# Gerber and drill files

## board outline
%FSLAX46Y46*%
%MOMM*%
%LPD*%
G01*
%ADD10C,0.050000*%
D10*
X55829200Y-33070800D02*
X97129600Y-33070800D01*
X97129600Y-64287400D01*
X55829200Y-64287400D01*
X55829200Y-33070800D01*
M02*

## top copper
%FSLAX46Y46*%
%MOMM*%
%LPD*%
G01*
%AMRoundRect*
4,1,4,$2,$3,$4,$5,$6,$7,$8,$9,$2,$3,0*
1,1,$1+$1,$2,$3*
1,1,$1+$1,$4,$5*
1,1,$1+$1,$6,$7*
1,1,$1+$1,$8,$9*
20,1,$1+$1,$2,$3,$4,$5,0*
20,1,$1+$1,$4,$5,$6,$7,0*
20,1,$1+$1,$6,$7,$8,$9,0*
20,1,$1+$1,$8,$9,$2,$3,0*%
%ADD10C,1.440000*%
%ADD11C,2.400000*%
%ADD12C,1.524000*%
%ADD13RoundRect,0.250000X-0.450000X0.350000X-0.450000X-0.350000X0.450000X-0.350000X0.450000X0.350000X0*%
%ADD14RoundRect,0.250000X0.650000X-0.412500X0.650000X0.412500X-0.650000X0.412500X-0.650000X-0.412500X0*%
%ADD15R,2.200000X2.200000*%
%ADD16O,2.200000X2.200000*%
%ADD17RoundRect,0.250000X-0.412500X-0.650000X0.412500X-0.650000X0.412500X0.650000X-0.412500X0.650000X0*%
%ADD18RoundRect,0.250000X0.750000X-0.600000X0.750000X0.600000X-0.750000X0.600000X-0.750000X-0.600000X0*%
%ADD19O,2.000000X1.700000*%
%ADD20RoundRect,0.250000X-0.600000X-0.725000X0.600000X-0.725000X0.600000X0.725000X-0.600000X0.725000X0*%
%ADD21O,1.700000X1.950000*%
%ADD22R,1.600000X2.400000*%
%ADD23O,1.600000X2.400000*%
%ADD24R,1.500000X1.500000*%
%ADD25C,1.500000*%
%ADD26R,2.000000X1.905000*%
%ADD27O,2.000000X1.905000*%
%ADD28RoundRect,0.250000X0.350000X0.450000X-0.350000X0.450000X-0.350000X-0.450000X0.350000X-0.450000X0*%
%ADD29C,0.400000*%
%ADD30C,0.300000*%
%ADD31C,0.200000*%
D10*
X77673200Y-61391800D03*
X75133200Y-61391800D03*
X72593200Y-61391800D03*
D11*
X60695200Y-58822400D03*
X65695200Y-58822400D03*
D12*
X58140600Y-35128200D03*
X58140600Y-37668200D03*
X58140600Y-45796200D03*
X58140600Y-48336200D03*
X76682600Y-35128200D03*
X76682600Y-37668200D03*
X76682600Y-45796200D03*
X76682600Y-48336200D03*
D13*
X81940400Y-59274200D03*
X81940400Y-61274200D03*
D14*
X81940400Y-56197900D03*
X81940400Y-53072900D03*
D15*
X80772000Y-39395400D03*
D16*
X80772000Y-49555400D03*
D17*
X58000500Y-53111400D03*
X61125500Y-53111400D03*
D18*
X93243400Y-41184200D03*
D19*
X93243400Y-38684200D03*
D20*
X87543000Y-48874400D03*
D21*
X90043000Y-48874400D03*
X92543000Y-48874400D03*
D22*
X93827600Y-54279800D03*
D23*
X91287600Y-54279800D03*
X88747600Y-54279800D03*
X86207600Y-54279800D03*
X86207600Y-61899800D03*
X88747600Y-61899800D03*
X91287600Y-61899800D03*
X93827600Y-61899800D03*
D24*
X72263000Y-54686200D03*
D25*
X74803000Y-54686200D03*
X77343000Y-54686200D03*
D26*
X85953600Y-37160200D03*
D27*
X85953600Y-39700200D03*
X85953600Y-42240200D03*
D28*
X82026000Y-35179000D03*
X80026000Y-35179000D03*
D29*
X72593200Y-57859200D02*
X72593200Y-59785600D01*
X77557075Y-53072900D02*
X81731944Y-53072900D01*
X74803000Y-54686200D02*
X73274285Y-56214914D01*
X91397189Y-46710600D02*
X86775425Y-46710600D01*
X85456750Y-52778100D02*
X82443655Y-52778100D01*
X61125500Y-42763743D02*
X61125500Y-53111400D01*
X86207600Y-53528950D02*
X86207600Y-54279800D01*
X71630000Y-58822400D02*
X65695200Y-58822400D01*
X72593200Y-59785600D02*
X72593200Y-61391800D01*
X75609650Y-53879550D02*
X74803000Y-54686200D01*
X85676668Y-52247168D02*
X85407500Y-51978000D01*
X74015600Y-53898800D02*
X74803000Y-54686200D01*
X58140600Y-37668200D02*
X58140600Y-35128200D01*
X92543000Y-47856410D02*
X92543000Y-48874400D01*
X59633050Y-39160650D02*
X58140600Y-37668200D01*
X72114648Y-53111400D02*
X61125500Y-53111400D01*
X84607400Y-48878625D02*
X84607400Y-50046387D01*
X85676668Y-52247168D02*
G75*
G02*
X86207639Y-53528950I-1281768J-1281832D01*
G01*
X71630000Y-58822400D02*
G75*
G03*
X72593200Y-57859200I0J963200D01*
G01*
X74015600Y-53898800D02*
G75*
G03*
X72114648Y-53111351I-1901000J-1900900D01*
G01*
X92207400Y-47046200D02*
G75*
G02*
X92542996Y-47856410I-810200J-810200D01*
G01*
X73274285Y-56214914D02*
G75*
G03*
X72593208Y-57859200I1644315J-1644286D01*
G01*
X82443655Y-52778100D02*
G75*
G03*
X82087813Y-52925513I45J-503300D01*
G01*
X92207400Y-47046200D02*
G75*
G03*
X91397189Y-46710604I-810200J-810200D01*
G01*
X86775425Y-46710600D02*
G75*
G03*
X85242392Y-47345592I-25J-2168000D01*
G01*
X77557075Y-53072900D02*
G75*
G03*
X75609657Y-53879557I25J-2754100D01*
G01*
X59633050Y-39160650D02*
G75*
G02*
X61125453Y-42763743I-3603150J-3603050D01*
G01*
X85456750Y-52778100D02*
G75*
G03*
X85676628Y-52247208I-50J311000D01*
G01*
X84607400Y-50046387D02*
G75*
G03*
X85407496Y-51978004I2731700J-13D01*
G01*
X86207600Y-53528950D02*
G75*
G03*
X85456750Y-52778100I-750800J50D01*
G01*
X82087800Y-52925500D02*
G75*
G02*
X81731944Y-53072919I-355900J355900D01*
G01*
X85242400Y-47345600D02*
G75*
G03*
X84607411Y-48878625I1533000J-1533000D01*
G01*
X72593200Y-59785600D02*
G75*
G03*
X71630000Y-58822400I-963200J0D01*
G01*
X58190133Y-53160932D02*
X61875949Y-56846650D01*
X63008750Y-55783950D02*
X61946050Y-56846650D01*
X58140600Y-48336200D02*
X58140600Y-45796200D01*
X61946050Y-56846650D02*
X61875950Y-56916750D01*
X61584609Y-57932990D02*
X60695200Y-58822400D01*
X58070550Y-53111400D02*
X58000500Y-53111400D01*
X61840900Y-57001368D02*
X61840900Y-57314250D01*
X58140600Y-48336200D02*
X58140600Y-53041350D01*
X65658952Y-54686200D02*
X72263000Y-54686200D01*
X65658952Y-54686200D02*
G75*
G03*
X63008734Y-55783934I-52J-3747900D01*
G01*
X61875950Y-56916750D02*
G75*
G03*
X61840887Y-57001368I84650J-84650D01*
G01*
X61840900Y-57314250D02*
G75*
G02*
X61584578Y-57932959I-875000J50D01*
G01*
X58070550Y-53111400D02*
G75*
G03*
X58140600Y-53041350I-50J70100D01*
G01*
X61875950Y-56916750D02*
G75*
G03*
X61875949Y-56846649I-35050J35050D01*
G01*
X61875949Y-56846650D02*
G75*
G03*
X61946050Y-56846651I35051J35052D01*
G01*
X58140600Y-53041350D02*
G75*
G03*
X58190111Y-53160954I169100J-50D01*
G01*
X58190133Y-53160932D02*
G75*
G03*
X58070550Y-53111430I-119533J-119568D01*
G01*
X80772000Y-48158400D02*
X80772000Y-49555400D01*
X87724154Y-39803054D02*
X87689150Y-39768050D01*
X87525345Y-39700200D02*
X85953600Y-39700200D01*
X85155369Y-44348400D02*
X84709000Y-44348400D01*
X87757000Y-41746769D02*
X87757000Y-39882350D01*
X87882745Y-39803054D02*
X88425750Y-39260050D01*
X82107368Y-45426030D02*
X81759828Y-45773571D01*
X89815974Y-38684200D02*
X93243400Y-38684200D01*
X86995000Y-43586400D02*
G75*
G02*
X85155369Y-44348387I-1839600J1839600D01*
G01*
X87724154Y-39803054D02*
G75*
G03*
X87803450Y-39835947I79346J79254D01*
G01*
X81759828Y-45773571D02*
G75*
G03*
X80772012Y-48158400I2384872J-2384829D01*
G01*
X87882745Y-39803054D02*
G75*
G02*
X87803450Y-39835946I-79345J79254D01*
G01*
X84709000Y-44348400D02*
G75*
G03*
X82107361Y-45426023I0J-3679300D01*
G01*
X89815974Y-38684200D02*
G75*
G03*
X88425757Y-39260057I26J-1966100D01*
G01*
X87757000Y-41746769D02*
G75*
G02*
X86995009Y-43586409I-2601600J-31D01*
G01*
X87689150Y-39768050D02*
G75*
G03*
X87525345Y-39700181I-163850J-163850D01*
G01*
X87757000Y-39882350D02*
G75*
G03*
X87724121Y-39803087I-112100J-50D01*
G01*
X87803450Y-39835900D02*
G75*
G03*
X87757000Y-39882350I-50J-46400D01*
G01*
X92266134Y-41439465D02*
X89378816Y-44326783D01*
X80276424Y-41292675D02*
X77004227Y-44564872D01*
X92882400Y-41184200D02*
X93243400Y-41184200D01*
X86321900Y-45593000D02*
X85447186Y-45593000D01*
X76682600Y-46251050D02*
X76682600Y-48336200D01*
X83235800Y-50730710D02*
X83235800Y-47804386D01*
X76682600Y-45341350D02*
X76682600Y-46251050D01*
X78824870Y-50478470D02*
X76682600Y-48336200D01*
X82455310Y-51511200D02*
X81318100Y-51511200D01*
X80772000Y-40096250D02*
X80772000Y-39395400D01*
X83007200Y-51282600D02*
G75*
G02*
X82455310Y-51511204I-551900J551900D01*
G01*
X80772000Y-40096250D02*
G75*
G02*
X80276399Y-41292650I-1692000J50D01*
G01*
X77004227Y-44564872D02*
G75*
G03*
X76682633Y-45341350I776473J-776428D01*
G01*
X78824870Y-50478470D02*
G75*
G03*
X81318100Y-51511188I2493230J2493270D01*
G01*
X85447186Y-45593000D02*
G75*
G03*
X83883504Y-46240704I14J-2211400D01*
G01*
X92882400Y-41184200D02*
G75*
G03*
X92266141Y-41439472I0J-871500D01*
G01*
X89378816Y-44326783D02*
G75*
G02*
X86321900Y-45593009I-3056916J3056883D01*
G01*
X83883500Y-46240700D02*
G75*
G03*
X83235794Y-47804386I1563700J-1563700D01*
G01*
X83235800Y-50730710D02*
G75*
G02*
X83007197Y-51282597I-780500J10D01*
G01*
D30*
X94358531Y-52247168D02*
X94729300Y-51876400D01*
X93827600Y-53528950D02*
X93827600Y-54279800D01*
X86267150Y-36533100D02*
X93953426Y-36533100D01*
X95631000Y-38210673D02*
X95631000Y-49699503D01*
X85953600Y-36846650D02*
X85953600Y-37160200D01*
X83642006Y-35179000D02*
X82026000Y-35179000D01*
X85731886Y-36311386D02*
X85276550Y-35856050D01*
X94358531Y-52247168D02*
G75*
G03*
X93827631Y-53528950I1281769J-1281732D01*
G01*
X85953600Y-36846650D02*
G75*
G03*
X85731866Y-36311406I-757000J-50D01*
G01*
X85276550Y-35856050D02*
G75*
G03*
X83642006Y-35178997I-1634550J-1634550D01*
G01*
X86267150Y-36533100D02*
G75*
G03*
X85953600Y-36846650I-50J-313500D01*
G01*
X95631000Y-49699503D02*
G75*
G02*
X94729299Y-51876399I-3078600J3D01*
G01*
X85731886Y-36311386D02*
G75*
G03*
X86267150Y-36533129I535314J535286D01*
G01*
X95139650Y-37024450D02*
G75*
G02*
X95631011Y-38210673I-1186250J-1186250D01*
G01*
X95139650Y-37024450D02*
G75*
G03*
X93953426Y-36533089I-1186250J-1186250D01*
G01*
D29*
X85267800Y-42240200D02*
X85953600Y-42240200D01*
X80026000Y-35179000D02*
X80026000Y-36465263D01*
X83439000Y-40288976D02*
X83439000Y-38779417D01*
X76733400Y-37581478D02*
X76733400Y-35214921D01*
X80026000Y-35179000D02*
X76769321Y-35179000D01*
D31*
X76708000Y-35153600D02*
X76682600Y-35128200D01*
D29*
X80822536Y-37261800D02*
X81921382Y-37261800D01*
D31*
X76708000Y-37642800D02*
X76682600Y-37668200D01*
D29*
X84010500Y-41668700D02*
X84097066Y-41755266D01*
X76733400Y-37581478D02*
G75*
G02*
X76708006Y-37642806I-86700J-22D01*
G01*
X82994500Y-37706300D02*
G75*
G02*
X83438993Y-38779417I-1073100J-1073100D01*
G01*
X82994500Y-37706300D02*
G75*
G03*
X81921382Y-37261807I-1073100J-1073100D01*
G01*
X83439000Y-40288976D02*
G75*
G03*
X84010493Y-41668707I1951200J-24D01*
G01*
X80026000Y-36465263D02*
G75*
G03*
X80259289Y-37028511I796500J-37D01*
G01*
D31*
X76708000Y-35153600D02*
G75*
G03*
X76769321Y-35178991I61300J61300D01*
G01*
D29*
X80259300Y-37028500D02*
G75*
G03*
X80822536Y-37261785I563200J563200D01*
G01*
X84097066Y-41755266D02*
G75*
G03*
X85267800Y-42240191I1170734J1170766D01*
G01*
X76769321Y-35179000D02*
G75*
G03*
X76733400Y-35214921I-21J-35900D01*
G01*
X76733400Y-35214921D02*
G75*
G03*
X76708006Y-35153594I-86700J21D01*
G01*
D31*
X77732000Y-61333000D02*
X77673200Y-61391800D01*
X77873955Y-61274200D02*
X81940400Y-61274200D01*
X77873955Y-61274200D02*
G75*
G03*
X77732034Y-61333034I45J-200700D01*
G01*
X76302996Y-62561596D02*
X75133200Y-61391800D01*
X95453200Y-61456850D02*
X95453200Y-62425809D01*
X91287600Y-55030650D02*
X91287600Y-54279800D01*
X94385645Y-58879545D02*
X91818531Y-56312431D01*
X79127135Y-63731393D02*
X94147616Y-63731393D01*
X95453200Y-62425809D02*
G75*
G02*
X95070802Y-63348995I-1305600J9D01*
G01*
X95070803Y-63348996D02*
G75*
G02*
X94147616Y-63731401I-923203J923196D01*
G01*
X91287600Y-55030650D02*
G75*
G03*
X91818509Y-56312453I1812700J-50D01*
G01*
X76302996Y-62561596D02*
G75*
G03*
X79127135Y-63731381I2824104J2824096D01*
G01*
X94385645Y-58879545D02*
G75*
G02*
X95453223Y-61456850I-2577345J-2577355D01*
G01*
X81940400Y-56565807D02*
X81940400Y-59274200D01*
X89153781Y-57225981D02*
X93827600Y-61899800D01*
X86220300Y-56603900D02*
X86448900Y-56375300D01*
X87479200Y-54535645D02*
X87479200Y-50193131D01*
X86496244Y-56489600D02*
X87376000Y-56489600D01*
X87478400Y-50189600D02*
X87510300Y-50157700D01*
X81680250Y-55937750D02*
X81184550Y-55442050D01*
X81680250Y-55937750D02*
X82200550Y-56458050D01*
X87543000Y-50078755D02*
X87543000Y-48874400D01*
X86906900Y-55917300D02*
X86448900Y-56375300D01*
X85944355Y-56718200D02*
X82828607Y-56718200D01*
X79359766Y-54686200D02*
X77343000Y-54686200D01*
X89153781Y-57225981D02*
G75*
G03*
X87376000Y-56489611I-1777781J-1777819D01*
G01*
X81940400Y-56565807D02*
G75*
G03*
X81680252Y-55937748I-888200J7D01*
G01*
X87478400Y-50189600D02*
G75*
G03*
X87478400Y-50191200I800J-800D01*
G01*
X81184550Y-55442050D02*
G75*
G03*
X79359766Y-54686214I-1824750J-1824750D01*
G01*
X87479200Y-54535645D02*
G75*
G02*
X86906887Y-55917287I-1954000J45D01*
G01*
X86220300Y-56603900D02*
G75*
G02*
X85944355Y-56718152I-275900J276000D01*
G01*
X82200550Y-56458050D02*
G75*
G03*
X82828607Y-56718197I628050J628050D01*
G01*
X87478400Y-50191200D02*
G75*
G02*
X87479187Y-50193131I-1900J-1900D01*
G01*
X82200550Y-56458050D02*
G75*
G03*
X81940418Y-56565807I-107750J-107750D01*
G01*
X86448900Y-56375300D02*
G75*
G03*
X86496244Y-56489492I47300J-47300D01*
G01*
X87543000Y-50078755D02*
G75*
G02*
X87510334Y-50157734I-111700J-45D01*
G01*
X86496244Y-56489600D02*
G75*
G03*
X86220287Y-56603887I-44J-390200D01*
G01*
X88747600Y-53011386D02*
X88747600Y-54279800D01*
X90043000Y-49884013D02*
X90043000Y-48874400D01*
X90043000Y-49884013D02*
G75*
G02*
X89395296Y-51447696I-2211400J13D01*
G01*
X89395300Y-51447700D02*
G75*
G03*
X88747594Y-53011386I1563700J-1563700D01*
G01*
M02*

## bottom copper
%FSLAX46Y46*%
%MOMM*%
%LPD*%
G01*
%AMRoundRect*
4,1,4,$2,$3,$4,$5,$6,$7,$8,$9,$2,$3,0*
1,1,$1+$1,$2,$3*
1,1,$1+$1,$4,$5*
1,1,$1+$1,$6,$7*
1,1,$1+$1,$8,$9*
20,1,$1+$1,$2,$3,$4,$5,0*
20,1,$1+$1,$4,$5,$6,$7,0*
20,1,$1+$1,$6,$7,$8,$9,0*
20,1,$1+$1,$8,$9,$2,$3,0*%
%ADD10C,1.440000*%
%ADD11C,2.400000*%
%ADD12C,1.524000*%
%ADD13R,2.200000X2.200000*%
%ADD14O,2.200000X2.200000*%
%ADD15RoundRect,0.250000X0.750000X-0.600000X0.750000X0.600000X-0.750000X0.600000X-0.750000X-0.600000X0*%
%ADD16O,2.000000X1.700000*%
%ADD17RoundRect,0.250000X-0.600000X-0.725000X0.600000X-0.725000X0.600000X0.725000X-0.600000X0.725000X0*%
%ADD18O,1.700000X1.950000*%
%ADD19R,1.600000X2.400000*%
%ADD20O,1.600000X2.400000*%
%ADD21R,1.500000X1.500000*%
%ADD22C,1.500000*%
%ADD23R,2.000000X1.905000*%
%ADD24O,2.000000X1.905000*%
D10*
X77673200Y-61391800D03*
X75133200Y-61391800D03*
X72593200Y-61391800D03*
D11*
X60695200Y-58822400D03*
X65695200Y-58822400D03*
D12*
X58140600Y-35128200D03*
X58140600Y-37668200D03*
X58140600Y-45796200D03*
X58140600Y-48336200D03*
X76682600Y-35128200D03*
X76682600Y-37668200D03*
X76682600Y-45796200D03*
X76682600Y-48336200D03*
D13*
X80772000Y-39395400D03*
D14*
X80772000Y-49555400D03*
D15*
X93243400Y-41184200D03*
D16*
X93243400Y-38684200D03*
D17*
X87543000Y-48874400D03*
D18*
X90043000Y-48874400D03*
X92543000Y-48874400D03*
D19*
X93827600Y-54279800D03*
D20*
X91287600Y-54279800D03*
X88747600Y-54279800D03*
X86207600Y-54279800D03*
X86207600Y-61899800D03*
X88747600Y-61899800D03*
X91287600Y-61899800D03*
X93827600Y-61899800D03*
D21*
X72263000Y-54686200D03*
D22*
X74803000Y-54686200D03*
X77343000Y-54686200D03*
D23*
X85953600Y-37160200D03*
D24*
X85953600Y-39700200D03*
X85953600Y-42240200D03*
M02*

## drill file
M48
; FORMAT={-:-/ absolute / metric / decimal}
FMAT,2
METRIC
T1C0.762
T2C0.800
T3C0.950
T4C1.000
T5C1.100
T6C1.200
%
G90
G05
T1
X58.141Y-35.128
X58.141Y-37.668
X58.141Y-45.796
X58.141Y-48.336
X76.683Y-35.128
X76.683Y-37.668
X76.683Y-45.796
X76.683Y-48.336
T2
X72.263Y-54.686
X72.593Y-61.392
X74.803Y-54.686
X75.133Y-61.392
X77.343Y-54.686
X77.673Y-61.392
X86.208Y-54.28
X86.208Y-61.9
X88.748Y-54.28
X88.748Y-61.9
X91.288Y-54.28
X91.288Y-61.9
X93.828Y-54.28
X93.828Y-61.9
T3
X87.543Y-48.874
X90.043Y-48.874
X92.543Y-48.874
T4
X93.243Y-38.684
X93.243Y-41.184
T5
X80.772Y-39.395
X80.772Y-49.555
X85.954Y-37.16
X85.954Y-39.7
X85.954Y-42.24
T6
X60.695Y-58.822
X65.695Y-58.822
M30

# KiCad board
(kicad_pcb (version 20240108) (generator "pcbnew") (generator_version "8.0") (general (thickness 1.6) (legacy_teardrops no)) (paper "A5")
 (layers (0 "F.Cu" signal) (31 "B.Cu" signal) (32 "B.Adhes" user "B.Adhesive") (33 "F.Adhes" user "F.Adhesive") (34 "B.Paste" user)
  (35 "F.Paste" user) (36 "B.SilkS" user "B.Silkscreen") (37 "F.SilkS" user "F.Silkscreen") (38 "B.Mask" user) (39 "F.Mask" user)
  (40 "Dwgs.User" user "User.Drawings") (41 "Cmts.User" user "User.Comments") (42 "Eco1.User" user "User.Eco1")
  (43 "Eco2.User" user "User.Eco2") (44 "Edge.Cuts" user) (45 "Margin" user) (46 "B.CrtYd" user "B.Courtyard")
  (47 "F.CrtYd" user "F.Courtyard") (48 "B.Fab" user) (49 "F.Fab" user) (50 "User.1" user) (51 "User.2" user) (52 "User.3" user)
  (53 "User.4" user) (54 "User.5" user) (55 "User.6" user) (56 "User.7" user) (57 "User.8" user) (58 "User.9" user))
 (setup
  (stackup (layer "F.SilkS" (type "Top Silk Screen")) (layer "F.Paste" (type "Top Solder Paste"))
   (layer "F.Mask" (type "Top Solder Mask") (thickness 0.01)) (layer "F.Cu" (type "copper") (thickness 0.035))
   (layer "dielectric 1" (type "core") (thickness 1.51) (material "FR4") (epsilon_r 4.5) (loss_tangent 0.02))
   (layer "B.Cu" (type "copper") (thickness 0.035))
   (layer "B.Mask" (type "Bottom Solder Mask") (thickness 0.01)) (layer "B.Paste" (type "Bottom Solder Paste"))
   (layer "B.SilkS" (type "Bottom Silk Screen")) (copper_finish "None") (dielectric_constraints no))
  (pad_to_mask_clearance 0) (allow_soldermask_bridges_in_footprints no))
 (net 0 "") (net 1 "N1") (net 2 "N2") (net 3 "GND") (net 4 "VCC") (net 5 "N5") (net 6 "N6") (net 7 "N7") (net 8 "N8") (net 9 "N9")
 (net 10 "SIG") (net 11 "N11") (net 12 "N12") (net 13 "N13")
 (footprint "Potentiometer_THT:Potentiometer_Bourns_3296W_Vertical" (layer "F.Cu") (at 77.6732 61.3918)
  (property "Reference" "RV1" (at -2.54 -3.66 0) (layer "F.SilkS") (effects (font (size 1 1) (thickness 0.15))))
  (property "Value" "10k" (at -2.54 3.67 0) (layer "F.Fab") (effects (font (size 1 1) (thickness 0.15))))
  (pad "1" thru_hole circle (at 0 0) (size 1.44 1.44) (drill 0.8) (layers "*.Cu" "*.Mask") (remove_unused_layers no) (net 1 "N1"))
  (pad "2" thru_hole circle (at -2.54 0) (size 1.44 1.44) (drill 0.8) (layers "*.Cu" "*.Mask") (remove_unused_layers no) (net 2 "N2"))
  (pad "3" thru_hole circle (at -5.08 0) (size 1.44 1.44) (drill 0.8) (layers "*.Cu" "*.Mask") (remove_unused_layers no) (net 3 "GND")))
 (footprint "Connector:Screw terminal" (layer "F.Cu") (at 63.1952 58.9224)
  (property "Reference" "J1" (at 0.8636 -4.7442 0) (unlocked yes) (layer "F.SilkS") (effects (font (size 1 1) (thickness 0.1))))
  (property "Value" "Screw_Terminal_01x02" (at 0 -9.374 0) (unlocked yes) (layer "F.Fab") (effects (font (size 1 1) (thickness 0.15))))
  (pad "1" thru_hole circle (at -2.5 -0.1) (size 2.4 2.4) (drill 1.2) (layers "*.Cu" "*.Mask") (remove_unused_layers no) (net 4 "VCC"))
  (pad "2" thru_hole circle (at 2.5 -0.1) (size 2.4 2.4) (drill 1.2) (layers "*.Cu" "*.Mask") (remove_unused_layers no) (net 3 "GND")))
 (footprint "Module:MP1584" (layer "F.Cu") (at 69.0626 41.2242)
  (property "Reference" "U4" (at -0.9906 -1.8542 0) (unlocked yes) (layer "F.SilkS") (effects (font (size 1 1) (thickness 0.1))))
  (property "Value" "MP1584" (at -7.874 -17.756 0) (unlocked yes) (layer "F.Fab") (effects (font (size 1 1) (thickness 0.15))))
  (pad "1" thru_hole circle (at -10.922 -6.096) (size 1.524 1.524) (drill 0.762) (layers "*.Cu" "*.Mask") (remove_unused_layers no)
   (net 3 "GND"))
  (pad "1" thru_hole circle (at -10.922 -3.556) (size 1.524 1.524) (drill 0.762) (layers "*.Cu" "*.Mask") (remove_unused_layers no)
   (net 3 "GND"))
  (pad "2" thru_hole circle (at -10.922 4.572) (size 1.524 1.524) (drill 0.762) (layers "*.Cu" "*.Mask") (remove_unused_layers no)
   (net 4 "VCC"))
  (pad "2" thru_hole circle (at -10.922 7.112) (size 1.524 1.524) (drill 0.762) (layers "*.Cu" "*.Mask") (remove_unused_layers no)
   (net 4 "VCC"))
  (pad "3" thru_hole circle (at 7.62 -6.096) (size 1.524 1.524) (drill 0.762) (layers "*.Cu" "*.Mask") (remove_unused_layers no)
   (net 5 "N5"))
  (pad "3" thru_hole circle (at 7.62 -3.556) (size 1.524 1.524) (drill 0.762) (layers "*.Cu" "*.Mask") (remove_unused_layers no)
   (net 5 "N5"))
  (pad "4" thru_hole circle (at 7.62 4.572) (size 1.524 1.524) (drill 0.762) (layers "*.Cu" "*.Mask") (remove_unused_layers no) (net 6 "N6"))
  (pad "4" thru_hole circle (at 7.62 7.112) (size 1.524 1.524) (drill 0.762) (layers "*.Cu" "*.Mask") (remove_unused_layers no) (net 6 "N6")))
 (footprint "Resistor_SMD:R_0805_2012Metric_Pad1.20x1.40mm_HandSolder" (layer "F.Cu") (at 81.9404 60.2742 -90)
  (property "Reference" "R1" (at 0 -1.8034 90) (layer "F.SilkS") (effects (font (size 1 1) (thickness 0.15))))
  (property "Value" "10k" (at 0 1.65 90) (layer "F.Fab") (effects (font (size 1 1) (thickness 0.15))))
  (pad "1" smd roundrect (at -1 0 270) (size 1.2 1.4) (layers "F.Cu" "F.Paste" "F.Mask") (roundrect_rratio 0.208333) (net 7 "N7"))
  (pad "2" smd roundrect (at 1 0 270) (size 1.2 1.4) (layers "F.Cu" "F.Paste" "F.Mask") (roundrect_rratio 0.208333) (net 1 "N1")))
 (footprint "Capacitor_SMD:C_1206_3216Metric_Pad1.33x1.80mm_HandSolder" (layer "F.Cu") (at 81.9404 54.6354 90)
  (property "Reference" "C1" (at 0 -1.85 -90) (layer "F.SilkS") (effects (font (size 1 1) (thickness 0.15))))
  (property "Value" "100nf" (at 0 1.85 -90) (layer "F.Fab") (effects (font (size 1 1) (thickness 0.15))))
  (pad "1" smd roundrect (at -1.5625 0 90) (size 1.325 1.8) (layers "F.Cu" "F.Paste" "F.Mask") (roundrect_rratio 0.188679) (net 7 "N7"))
  (pad "2" smd roundrect (at 1.5625 0 90) (size 1.325 1.8) (layers "F.Cu" "F.Paste" "F.Mask") (roundrect_rratio 0.188679) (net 3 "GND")))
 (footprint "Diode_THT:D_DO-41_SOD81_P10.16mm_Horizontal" (layer "F.Cu") (at 80.772 39.3954 -90)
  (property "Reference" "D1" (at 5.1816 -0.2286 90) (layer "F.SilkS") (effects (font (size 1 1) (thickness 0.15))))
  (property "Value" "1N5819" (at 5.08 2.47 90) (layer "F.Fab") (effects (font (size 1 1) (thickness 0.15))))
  (pad "1" thru_hole rect (at 0 0 270) (size 2.2 2.2) (drill 1.1) (layers "*.Cu" "*.Mask") (remove_unused_layers no) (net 6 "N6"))
  (pad "2" thru_hole oval (at 10.16 0 270) (size 2.2 2.2) (drill 1.1) (layers "*.Cu" "*.Mask") (remove_unused_layers no) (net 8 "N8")))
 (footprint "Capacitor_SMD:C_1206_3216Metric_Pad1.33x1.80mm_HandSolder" (layer "F.Cu") (at 59.563 53.1114)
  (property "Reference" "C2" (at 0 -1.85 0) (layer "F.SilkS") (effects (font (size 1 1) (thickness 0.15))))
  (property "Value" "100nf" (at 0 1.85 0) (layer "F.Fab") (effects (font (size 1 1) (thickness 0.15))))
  (pad "1" smd roundrect (at -1.5625 0) (size 1.325 1.8) (layers "F.Cu" "F.Paste" "F.Mask") (roundrect_rratio 0.188679) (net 4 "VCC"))
  (pad "2" smd roundrect (at 1.5625 0) (size 1.325 1.8) (layers "F.Cu" "F.Paste" "F.Mask") (roundrect_rratio 0.188679) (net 3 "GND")))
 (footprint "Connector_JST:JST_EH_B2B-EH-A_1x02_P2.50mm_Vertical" (layer "F.Cu") (at 93.2434 41.1842 90)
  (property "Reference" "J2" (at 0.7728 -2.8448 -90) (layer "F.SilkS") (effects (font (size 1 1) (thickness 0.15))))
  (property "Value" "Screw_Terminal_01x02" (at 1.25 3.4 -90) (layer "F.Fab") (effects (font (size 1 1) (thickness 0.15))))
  (pad "1" thru_hole roundrect (at 0 0 90) (size 1.7 2) (drill 1) (layers "*.Cu" "*.Mask") (remove_unused_layers no)
   (roundrect_rratio 0.147059) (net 6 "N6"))
  (pad "2" thru_hole oval (at 2.5 0 90) (size 1.7 2) (drill 1) (layers "*.Cu" "*.Mask") (remove_unused_layers no) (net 8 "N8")))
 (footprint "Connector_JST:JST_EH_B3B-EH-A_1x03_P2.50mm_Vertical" (layer "F.Cu") (at 87.543 48.8744)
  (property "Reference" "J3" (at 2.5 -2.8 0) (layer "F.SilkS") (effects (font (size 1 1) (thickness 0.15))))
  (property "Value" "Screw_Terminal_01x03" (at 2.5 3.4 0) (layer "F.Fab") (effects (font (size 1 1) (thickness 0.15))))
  (pad "1" thru_hole roundrect (at 0 0) (size 1.7 1.95) (drill 0.95) (layers "*.Cu" "*.Mask") (remove_unused_layers no)
   (roundrect_rratio 0.147059) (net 7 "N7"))
  (pad "2" thru_hole oval (at 2.5 0) (size 1.7 1.95) (drill 0.95) (layers "*.Cu" "*.Mask") (remove_unused_layers no) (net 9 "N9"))
  (pad "3" thru_hole oval (at 5 0) (size 1.7 1.95) (drill 0.95) (layers "*.Cu" "*.Mask") (remove_unused_layers no) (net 3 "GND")))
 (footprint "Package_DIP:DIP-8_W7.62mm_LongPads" (layer "F.Cu") (at 93.8276 54.2798 -90)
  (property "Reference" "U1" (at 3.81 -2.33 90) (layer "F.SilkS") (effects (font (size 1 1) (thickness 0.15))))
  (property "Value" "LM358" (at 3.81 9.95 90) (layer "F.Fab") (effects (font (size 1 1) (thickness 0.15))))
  (pad "1" thru_hole rect (at 0 0 270) (size 2.4 1.6) (drill 0.8) (layers "*.Cu" "*.Mask") (remove_unused_layers no) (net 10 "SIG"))
  (pad "2" thru_hole oval (at 0 2.54 270) (size 2.4 1.6) (drill 0.8) (layers "*.Cu" "*.Mask") (remove_unused_layers no) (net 2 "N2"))
  (pad "3" thru_hole oval (at 0 5.08 270) (size 2.4 1.6) (drill 0.8) (layers "*.Cu" "*.Mask") (remove_unused_layers no) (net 9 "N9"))
  (pad "4" thru_hole oval (at 0 7.62 270) (size 2.4 1.6) (drill 0.8) (layers "*.Cu" "*.Mask") (remove_unused_layers no) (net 3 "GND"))
  (pad "5" thru_hole oval (at 7.62 7.62 270) (size 2.4 1.6) (drill 0.8) (layers "*.Cu" "*.Mask") (remove_unused_layers no) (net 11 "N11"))
  (pad "6" thru_hole oval (at 7.62 5.08 270) (size 2.4 1.6) (drill 0.8) (layers "*.Cu" "*.Mask") (remove_unused_layers no) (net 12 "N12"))
  (pad "7" thru_hole oval (at 7.62 2.54 270) (size 2.4 1.6) (drill 0.8) (layers "*.Cu" "*.Mask") (remove_unused_layers no) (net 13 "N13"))
  (pad "8" thru_hole oval (at 7.62 0 270) (size 2.4 1.6) (drill 0.8) (layers "*.Cu" "*.Mask") (remove_unused_layers no) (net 7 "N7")))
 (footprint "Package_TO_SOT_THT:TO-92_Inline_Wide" (layer "F.Cu") (at 72.263 54.6862)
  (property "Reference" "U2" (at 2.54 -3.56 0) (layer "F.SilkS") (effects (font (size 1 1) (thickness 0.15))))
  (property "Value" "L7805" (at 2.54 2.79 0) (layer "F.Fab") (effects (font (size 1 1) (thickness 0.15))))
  (pad "1" thru_hole rect (at 0 0) (size 1.5 1.5) (drill 0.8) (layers "*.Cu" "*.Mask") (remove_unused_layers no) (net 4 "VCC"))
  (pad "2" thru_hole circle (at 2.54 0) (size 1.5 1.5) (drill 0.8) (layers "*.Cu" "*.Mask") (remove_unused_layers no) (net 3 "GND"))
  (pad "3" thru_hole circle (at 5.08 0) (size 1.5 1.5) (drill 0.8) (layers "*.Cu" "*.Mask") (remove_unused_layers no) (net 7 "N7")))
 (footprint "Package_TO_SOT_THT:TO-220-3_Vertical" (layer "F.Cu") (at 85.9536 37.1602 -90)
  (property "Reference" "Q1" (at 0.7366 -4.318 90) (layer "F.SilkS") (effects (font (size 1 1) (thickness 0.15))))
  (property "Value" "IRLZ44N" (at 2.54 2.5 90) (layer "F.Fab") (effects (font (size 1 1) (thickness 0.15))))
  (pad "1" thru_hole rect (at 0 0 270) (size 1.905 2) (drill 1.1) (layers "*.Cu" "*.Mask") (remove_unused_layers no) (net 10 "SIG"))
  (pad "2" thru_hole oval (at 2.54 0 270) (size 1.905 2) (drill 1.1) (layers "*.Cu" "*.Mask") (remove_unused_layers no) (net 8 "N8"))
  (pad "3" thru_hole oval (at 5.08 0 270) (size 1.905 2) (drill 1.1) (layers "*.Cu" "*.Mask") (remove_unused_layers no) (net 5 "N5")))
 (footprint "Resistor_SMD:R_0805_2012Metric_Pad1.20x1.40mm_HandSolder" (layer "F.Cu") (at 81.026 35.179 180)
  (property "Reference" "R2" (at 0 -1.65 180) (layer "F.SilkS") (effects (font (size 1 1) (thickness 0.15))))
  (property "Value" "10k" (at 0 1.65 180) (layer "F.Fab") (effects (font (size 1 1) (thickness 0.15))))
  (pad "1" smd roundrect (at -1 0 180) (size 1.2 1.4) (layers "F.Cu" "F.Paste" "F.Mask") (roundrect_rratio 0.208333) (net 10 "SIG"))
  (pad "2" smd roundrect (at 1 0 180) (size 1.2 1.4) (layers "F.Cu" "F.Paste" "F.Mask") (roundrect_rratio 0.208333) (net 5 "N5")))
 (gr_rect (start 55.8292 33.0708) (end 97.1296 64.2874) (stroke (width 0.05) (type default)) (fill none) (layer "Edge.Cuts"))
 (segment (start 72.5932 57.8592) (end 72.5932 59.7856) (width 0.4) (layer "F.Cu") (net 3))
 (segment (start 77.557075 53.0729) (end 81.731944 53.0729) (width 0.4) (layer "F.Cu") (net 3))
 (segment (start 74.803 54.6862) (end 73.274285 56.214914) (width 0.4) (layer "F.Cu") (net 3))
 (segment (start 91.397189 46.7106) (end 86.775425 46.7106) (width 0.4) (layer "F.Cu") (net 3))
 (segment (start 85.45675 52.7781) (end 82.443655 52.7781) (width 0.4) (layer "F.Cu") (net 3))
 (segment (start 61.1255 42.763743) (end 61.1255 53.1114) (width 0.4) (layer "F.Cu") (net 3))
 (segment (start 86.2076 53.52895) (end 86.2076 54.2798) (width 0.4) (layer "F.Cu") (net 3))
 (segment (start 71.63 58.8224) (end 65.6952 58.8224) (width 0.4) (layer "F.Cu") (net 3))
 (segment (start 72.5932 59.7856) (end 72.5932 61.3918) (width 0.4) (layer "F.Cu") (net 3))
 (segment (start 75.60965 53.87955) (end 74.803 54.6862) (width 0.4) (layer "F.Cu") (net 3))
 (segment (start 85.676668 52.247168) (end 85.4075 51.978) (width 0.4) (layer "F.Cu") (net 3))
 (segment (start 74.0156 53.8988) (end 74.803 54.6862) (width 0.4) (layer "F.Cu") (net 3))
 (segment (start 58.1406 37.6682) (end 58.1406 35.1282) (width 0.4) (layer "F.Cu") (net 3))
 (segment (start 92.543 47.85641) (end 92.543 48.8744) (width 0.4) (layer "F.Cu") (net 3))
 (segment (start 59.63305 39.16065) (end 58.1406 37.6682) (width 0.4) (layer "F.Cu") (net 3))
 (segment (start 72.114648 53.1114) (end 61.1255 53.1114) (width 0.4) (layer "F.Cu") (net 3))
 (segment (start 84.6074 48.878625) (end 84.6074 50.046387) (width 0.4) (layer "F.Cu") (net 3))
 (arc (start 85.676668 52.247168) (mid 86.069615 52.835254) (end 86.2076 53.52895) (width 0.4) (layer "F.Cu") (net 3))
 (arc (start 71.63 58.8224) (mid 72.311085 58.540285) (end 72.5932 57.8592) (width 0.4) (layer "F.Cu") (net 3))
 (arc (start 74.0156 53.8988) (mid 73.143435 53.316038) (end 72.114648 53.1114) (width 0.4) (layer "F.Cu") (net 3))
 (arc (start 92.2074 47.0462) (mid 92.45578 47.417927) (end 92.543 47.85641) (width 0.4) (layer "F.Cu") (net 3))
 (arc (start 73.274285 56.214914) (mid 72.770208 56.969319) (end 72.5932 57.8592) (width 0.4) (layer "F.Cu") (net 3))
 (arc (start 82.443655 52.7781) (mid 82.251067 52.816408) (end 82.0878 52.9255) (width 0.4) (layer "F.Cu") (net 3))
 (arc (start 92.2074 47.0462) (mid 91.835672 46.797819) (end 91.397189 46.7106) (width 0.4) (layer "F.Cu") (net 3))
 (arc (start 86.775425 46.7106) (mid 85.945757 46.875631) (end 85.2424 47.3456) (width 0.4) (layer "F.Cu") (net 3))
 (arc (start 77.557075 53.0729) (mid 76.503136 53.282541) (end 75.60965 53.87955) (width 0.4) (layer "F.Cu") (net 3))
 (arc (start 59.63305 39.16065) (mid 60.737624 40.813763) (end 61.1255 42.763743) (width 0.4) (layer "F.Cu") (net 3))
 (arc (start 85.45675 52.7781) (mid 85.744087 52.586106) (end 85.676668 52.247168) (width 0.4) (layer "F.Cu") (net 3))
 (arc (start 84.6074 50.046387) (mid 84.815339 51.091768) (end 85.4075 51.978) (width 0.4) (layer "F.Cu") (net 3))
 (arc (start 86.2076 53.52895) (mid 85.987681 52.998018) (end 85.45675 52.7781) (width 0.4) (layer "F.Cu") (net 3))
 (arc (start 82.0878 52.9255) (mid 81.924532 53.034591) (end 81.731944 53.0729) (width 0.4) (layer "F.Cu") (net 3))
 (arc (start 85.2424 47.3456) (mid 84.772431 48.048957) (end 84.6074 48.878625) (width 0.4) (layer "F.Cu") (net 3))
 (arc (start 72.5932 59.7856) (mid 72.311085 59.104514) (end 71.63 58.8224) (width 0.4) (layer "F.Cu") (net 3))
 (segment (start 58.190133 53.160932) (end 61.875949 56.84665) (width 0.4) (layer "F.Cu") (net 4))
 (segment (start 63.00875 55.78395) (end 61.94605 56.84665) (width 0.4) (layer "F.Cu") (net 4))
 (segment (start 58.1406 48.3362) (end 58.1406 45.7962) (width 0.4) (layer "F.Cu") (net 4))
 (segment (start 61.94605 56.84665) (end 61.87595 56.91675) (width 0.4) (layer "F.Cu") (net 4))
 (segment (start 61.584609 57.93299) (end 60.6952 58.8224) (width 0.4) (layer "F.Cu") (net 4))
 (segment (start 58.07055 53.1114) (end 58.0005 53.1114) (width 0.4) (layer "F.Cu") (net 4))
 (segment (start 61.8409 57.001368) (end 61.8409 57.31425) (width 0.4) (layer "F.Cu") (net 4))
 (segment (start 58.1406 48.3362) (end 58.1406 53.04135) (width 0.4) (layer "F.Cu") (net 4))
 (segment (start 65.658952 54.6862) (end 72.263 54.6862) (width 0.4) (layer "F.Cu") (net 4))
 (arc (start 65.658952 54.6862) (mid 64.224673 54.971495) (end 63.00875 55.78395) (width 0.4) (layer "F.Cu") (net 4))
 (arc (start 61.87595 56.91675) (mid 61.850009 56.955573) (end 61.8409 57.001368) (width 0.4) (layer "F.Cu") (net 4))
 (arc (start 61.8409 57.31425) (mid 61.774292 57.649109) (end 61.584609 57.93299) (width 0.4) (layer "F.Cu") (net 4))
 (arc (start 58.07055 53.1114) (mid 58.120082 53.090882) (end 58.1406 53.04135) (width 0.4) (layer "F.Cu") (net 4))
 (arc (start 61.87595 56.91675) (mid 61.890467 56.8817) (end 61.875949 56.84665) (width 0.4) (layer "F.Cu") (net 4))
 (arc (start 61.875949 56.84665) (mid 61.910999 56.861168) (end 61.94605 56.84665) (width 0.4) (layer "F.Cu") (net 4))
 (arc (start 58.1406 53.04135) (mid 58.153473 53.106067) (end 58.190133 53.160932) (width 0.4) (layer "F.Cu") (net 4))
 (arc (start 58.190133 53.160932) (mid 58.135267 53.124272) (end 58.07055 53.1114) (width 0.4) (layer "F.Cu") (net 4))
 (segment (start 80.772 48.1584) (end 80.772 49.5554) (width 0.4) (layer "F.Cu") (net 8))
 (segment (start 87.724154 39.803054) (end 87.68915 39.76805) (width 0.4) (layer "F.Cu") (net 8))
 (segment (start 87.525345 39.7002) (end 85.9536 39.7002) (width 0.4) (layer "F.Cu") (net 8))
 (segment (start 85.155369 44.3484) (end 84.709 44.3484) (width 0.4) (layer "F.Cu") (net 8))
 (segment (start 87.757 41.746769) (end 87.757 39.88235) (width 0.4) (layer "F.Cu") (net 8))
 (segment (start 87.882745 39.803054) (end 88.42575 39.26005) (width 0.4) (layer "F.Cu") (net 8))
 (segment (start 82.107368 45.42603) (end 81.759828 45.773571) (width 0.4) (layer "F.Cu") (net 8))
 (segment (start 89.815974 38.6842) (end 93.2434 38.6842) (width 0.4) (layer "F.Cu") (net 8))
 (arc (start 86.995 43.5864) (mid 86.15097 44.150362) (end 85.155369 44.3484) (width 0.4) (layer "F.Cu") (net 8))
 (arc (start 87.724154 39.803054) (mid 87.760535 39.827363) (end 87.80345 39.8359) (width 0.4) (layer "F.Cu") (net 8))
 (arc (start 81.759828 45.773571) (mid 81.028728 46.86774) (end 80.772 48.1584) (width 0.4) (layer "F.Cu") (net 8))
 (arc (start 87.882745 39.803054) (mid 87.846364 39.827363) (end 87.80345 39.8359) (width 0.4) (layer "F.Cu") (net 8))
 (arc (start 84.709 44.3484) (mid 83.301007 44.628466) (end 82.107368 45.42603) (width 0.4) (layer "F.Cu") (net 8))
 (arc (start 89.815974 38.6842) (mid 89.06359 38.833858) (end 88.42575 39.26005) (width 0.4) (layer "F.Cu") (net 8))
 (arc (start 87.757 41.746769) (mid 87.558962 42.74237) (end 86.995 43.5864) (width 0.4) (layer "F.Cu") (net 8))
 (arc (start 87.68915 39.76805) (mid 87.613995 39.717833) (end 87.525345 39.7002) (width 0.4) (layer "F.Cu") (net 8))
 (arc (start 87.757 39.88235) (mid 87.748463 39.839435) (end 87.724154 39.803054) (width 0.4) (layer "F.Cu") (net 8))
 (arc (start 87.80345 39.8359) (mid 87.770604 39.849504) (end 87.757 39.88235) (width 0.4) (layer "F.Cu") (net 8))
 (segment (start 92.266134 41.439465) (end 89.378816 44.326783) (width 0.4) (layer "F.Cu") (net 6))
 (segment (start 80.276424 41.292675) (end 77.004227 44.564872) (width 0.4) (layer "F.Cu") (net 6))
 (segment (start 92.8824 41.1842) (end 93.2434 41.1842) (width 0.4) (layer "F.Cu") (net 6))
 (segment (start 86.3219 45.593) (end 85.447186 45.593) (width 0.4) (layer "F.Cu") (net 6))
 (segment (start 76.6826 46.25105) (end 76.6826 48.3362) (width 0.4) (layer "F.Cu") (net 6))
 (segment (start 83.2358 50.73071) (end 83.2358 47.804386) (width 0.4) (layer "F.Cu") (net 6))
 (segment (start 76.6826 45.34135) (end 76.6826 46.25105) (width 0.4) (layer "F.Cu") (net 6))
 (segment (start 78.82487 50.47847) (end 76.6826 48.3362) (width 0.4) (layer "F.Cu") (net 6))
 (segment (start 82.45531 51.5112) (end 81.3181 51.5112) (width 0.4) (layer "F.Cu") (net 6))
 (segment (start 80.772 40.09625) (end 80.772 39.3954) (width 0.4) (layer "F.Cu") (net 6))
 (arc (start 83.0072 51.2826) (mid 82.75399 51.451788) (end 82.45531 51.5112) (width 0.4) (layer "F.Cu") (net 6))
 (arc (start 80.772 40.09625) (mid 80.643203 40.74375) (end 80.276424 41.292675) (width 0.4) (layer "F.Cu") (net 6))
 (arc (start 77.004227 44.564872) (mid 76.766188 44.921123) (end 76.6826 45.34135) (width 0.4) (layer "F.Cu") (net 6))
 (arc (start 78.82487 50.47847) (mid 79.968773 51.242802) (end 81.3181 51.5112) (width 0.4) (layer "F.Cu") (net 6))
 (arc (start 85.447186 45.593) (mid 84.600925 45.761331) (end 83.8835 46.2407) (width 0.4) (layer "F.Cu") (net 6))
 (arc (start 92.8824 41.1842) (mid 92.548879 41.250541) (end 92.266134 41.439465) (width 0.4) (layer "F.Cu") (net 6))
 (arc (start 89.378816 44.326783) (mid 87.976291 45.26392) (end 86.3219 45.593) (width 0.4) (layer "F.Cu") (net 6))
 (arc (start 83.8835 46.2407) (mid 83.404131 46.958125) (end 83.2358 47.804386) (width 0.4) (layer "F.Cu") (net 6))
 (arc (start 83.2358 50.73071) (mid 83.176388 51.02939) (end 83.0072 51.2826) (width 0.4) (layer "F.Cu") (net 6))
 (segment (start 94.358531 52.247168) (end 94.7293 51.8764) (width 0.3) (layer "F.Cu") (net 10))
 (segment (start 93.8276 53.52895) (end 93.8276 54.2798) (width 0.3) (layer "F.Cu") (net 10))
 (segment (start 86.26715 36.5331) (end 93.953426 36.5331) (width 0.3) (layer "F.Cu") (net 10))
 (segment (start 95.631 38.210673) (end 95.631 49.699503) (width 0.3) (layer "F.Cu") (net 10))
 (segment (start 85.9536 36.84665) (end 85.9536 37.1602) (width 0.3) (layer "F.Cu") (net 10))
 (segment (start 83.642006 35.179) (end 82.026 35.179) (width 0.3) (layer "F.Cu") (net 10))
 (segment (start 85.731886 36.311386) (end 85.27655 35.85605) (width 0.3) (layer "F.Cu") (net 10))
 (arc (start 94.358531 52.247168) (mid 93.965584 52.835254) (end 93.8276 53.52895) (width 0.3) (layer "F.Cu") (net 10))
 (arc (start 85.9536 36.84665) (mid 85.895978 36.556967) (end 85.731886 36.311386) (width 0.3) (layer "F.Cu") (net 10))
 (arc (start 85.27655 35.85605) (mid 84.526614 35.354959) (end 83.642006 35.179) (width 0.3) (layer "F.Cu") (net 10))
 (arc (start 86.26715 36.5331) (mid 86.045436 36.624936) (end 85.9536 36.84665) (width 0.3) (layer "F.Cu") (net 10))
 (arc (start 95.631 49.699503) (mid 95.396655 50.877631) (end 94.7293 51.8764) (width 0.3) (layer "F.Cu") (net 10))
 (arc (start 85.731886 36.311386) (mid 85.977467 36.475478) (end 86.26715 36.5331) (width 0.3) (layer "F.Cu") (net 10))
 (arc (start 95.13965 37.02445) (mid 95.503302 37.568693) (end 95.631 38.210673) (width 0.3) (layer "F.Cu") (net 10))
 (arc (start 95.13965 37.02445) (mid 94.595405 36.660797) (end 93.953426 36.5331) (width 0.3) (layer "F.Cu") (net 10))
 (segment (start 85.2678 42.2402) (end 85.9536 42.2402) (width 0.4) (layer "F.Cu") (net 5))
 (segment (start 80.026 35.179) (end 80.026 36.465263) (width 0.4) (layer "F.Cu") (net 5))
 (segment (start 83.439 40.288976) (end 83.439 38.779417) (width 0.4) (layer "F.Cu") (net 5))
 (segment (start 76.7334 37.581478) (end 76.7334 35.214921) (width 0.4) (layer "F.Cu") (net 5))
 (segment (start 80.026 35.179) (end 76.769321 35.179) (width 0.4) (layer "F.Cu") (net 5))
 (segment (start 76.708 35.1536) (end 76.6826 35.1282) (width 0.2) (layer "F.Cu") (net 5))
 (segment (start 80.822536 37.2618) (end 81.921382 37.2618) (width 0.4) (layer "F.Cu") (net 5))
 (segment (start 76.708 37.6428) (end 76.6826 37.6682) (width 0.2) (layer "F.Cu") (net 5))
 (segment (start 84.0105 41.6687) (end 84.097066 41.755266) (width 0.4) (layer "F.Cu") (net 5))
 (arc (start 76.7334 37.581478) (mid 76.726798 37.614665) (end 76.708 37.6428) (width 0.4) (layer "F.Cu") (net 5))
 (arc (start 82.9945 37.7063) (mid 83.323478 38.19865) (end 83.439 38.779417) (width 0.4) (layer "F.Cu") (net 5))
 (arc (start 82.9945 37.7063) (mid 82.502149 37.377321) (end 81.921382 37.2618) (width 0.4) (layer "F.Cu") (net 5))
 (arc (start 83.439 40.288976) (mid 83.587528 41.035677) (end 84.0105 41.6687) (width 0.4) (layer "F.Cu") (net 5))
 (arc (start 80.026 36.465263) (mid 80.086632 36.770084) (end 80.2593 37.0285) (width 0.4) (layer "F.Cu") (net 5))
 (arc (start 76.708 35.1536) (mid 76.736134 35.172398) (end 76.769321 35.179) (width 0.2) (layer "F.Cu") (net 5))
 (arc (start 80.2593 37.0285) (mid 80.517714 37.201167) (end 80.822536 37.2618) (width 0.4) (layer "F.Cu") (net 5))
 (arc (start 84.097066 41.755266) (mid 84.634203 42.114169) (end 85.2678 42.2402) (width 0.4) (layer "F.Cu") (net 5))
 (arc (start 76.769321 35.179) (mid 76.743921 35.189521) (end 76.7334 35.214921) (width 0.4) (layer "F.Cu") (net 5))
 (arc (start 76.7334 35.214921) (mid 76.726798 35.181734) (end 76.708 35.1536) (width 0.4) (layer "F.Cu") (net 5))
 (segment (start 77.732 61.333) (end 77.6732 61.3918) (width 0.2) (layer "F.Cu") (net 1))
 (segment (start 77.873955 61.2742) (end 81.9404 61.2742) (width 0.2) (layer "F.Cu") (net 1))
 (arc (start 77.873955 61.2742) (mid 77.797129 61.289481) (end 77.732 61.333) (width 0.2) (layer "F.Cu") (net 1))
 (segment (start 76.302996 62.561596) (end 75.1332 61.3918) (width 0.2) (layer "F.Cu") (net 2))
 (segment (start 95.4532 61.45685) (end 95.4532 62.425809) (width 0.2) (layer "F.Cu") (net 2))
 (segment (start 91.2876 55.03065) (end 91.2876 54.2798) (width 0.2) (layer "F.Cu") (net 2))
 (segment (start 94.385645 58.879545) (end 91.818531 56.312431) (width 0.2) (layer "F.Cu") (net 2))
 (segment (start 79.127135 63.731393) (end 94.147616 63.731393) (width 0.2) (layer "F.Cu") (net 2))
 (arc (start 95.4532 62.425809) (mid 95.353818 62.925434) (end 95.070803 63.348996) (width 0.2) (layer "F.Cu") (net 2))
 (arc (start 95.070803 63.348996) (mid 94.647241 63.632011) (end 94.147616 63.731393) (width 0.2) (layer "F.Cu") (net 2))
 (arc (start 91.2876 55.03065) (mid 91.425584 55.724344) (end 91.818531 56.312431) (width 0.2) (layer "F.Cu") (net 2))
 (arc (start 76.302996 62.561596) (mid 77.598722 63.427372) (end 79.127135 63.731393) (width 0.2) (layer "F.Cu") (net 2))
 (arc (start 94.385645 58.879545) (mid 95.175751 60.062022) (end 95.4532 61.45685) (width 0.2) (layer "F.Cu") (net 2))
 (segment (start 81.9404 56.565807) (end 81.9404 59.2742) (width 0.2) (layer "F.Cu") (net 7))
 (segment (start 89.153781 57.225981) (end 93.8276 61.8998) (width 0.2) (layer "F.Cu") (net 7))
 (segment (start 86.2203 56.6039) (end 86.4489 56.3753) (width 0.2) (layer "F.Cu") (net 7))
 (segment (start 87.4792 54.535645) (end 87.4792 50.193131) (width 0.2) (layer "F.Cu") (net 7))
 (segment (start 86.496244 56.4896) (end 87.376 56.4896) (width 0.2) (layer "F.Cu") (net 7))
 (segment (start 87.4784 50.1896) (end 87.5103 50.1577) (width 0.2) (layer "F.Cu") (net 7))
 (segment (start 81.68025 55.93775) (end 81.18455 55.44205) (width 0.2) (layer "F.Cu") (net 7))
 (segment (start 81.68025 55.93775) (end 82.20055 56.45805) (width 0.2) (layer "F.Cu") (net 7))
 (segment (start 87.543 50.078755) (end 87.543 48.8744) (width 0.2) (layer "F.Cu") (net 7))
 (segment (start 86.9069 55.9173) (end 86.4489 56.3753) (width 0.2) (layer "F.Cu") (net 7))
 (segment (start 85.944355 56.7182) (end 82.828607 56.7182) (width 0.2) (layer "F.Cu") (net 7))
 (segment (start 79.359766 54.6862) (end 77.343 54.6862) (width 0.2) (layer "F.Cu") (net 7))
 (arc (start 89.153781 57.225981) (mid 88.338128 56.680979) (end 87.376 56.4896) (width 0.2) (layer "F.Cu") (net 7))
 (arc (start 81.9404 56.565807) (mid 81.872789 56.225905) (end 81.68025 55.93775) (width 0.2) (layer "F.Cu") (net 7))
 (arc (start 87.4784 50.1896) (mid 87.478068 50.1904) (end 87.4784 50.1912) (width 0.2) (layer "F.Cu") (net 7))
 (arc (start 81.18455 55.44205) (mid 80.347332 54.882639) (end 79.359766 54.6862) (width 0.2) (layer "F.Cu") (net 7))
 (arc (start 87.4792 54.535645) (mid 87.330464 55.283391) (end 86.9069 55.9173) (width 0.2) (layer "F.Cu") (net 7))
 (arc (start 86.2203 56.6039) (mid 86.093695 56.688494) (end 85.944355 56.7182) (width 0.2) (layer "F.Cu") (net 7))
 (arc (start 82.20055 56.45805) (mid 82.488705 56.650589) (end 82.828607 56.7182) (width 0.2) (layer "F.Cu") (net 7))
 (arc (start 87.4784 50.1912) (mid 87.478992 50.192086) (end 87.4792 50.193131) (width 0.2) (layer "F.Cu") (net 7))
 (arc (start 82.20055 56.45805) (mid 82.034474 56.425015) (end 81.9404 56.565807) (width 0.2) (layer "F.Cu") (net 7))
 (arc (start 86.4489 56.3753) (mid 86.434385 56.448267) (end 86.496244 56.4896) (width 0.2) (layer "F.Cu") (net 7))
 (arc (start 87.543 50.078755) (mid 87.534501 50.121479) (end 87.5103 50.1577) (width 0.2) (layer "F.Cu") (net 7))
 (arc (start 86.496244 56.4896) (mid 86.346904 56.519305) (end 86.2203 56.6039) (width 0.2) (layer "F.Cu") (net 7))
 (segment (start 88.7476 53.011386) (end 88.7476 54.2798) (width 0.2) (layer "F.Cu") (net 9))
 (segment (start 90.043 49.884013) (end 90.043 48.8744) (width 0.2) (layer "F.Cu") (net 9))
 (arc (start 90.043 49.884013) (mid 89.874668 50.730274) (end 89.3953 51.4477) (width 0.2) (layer "F.Cu") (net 9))
 (arc (start 89.3953 51.4477) (mid 88.915931 52.165125) (end 88.7476 53.011386) (width 0.2) (layer "F.Cu") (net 9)))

